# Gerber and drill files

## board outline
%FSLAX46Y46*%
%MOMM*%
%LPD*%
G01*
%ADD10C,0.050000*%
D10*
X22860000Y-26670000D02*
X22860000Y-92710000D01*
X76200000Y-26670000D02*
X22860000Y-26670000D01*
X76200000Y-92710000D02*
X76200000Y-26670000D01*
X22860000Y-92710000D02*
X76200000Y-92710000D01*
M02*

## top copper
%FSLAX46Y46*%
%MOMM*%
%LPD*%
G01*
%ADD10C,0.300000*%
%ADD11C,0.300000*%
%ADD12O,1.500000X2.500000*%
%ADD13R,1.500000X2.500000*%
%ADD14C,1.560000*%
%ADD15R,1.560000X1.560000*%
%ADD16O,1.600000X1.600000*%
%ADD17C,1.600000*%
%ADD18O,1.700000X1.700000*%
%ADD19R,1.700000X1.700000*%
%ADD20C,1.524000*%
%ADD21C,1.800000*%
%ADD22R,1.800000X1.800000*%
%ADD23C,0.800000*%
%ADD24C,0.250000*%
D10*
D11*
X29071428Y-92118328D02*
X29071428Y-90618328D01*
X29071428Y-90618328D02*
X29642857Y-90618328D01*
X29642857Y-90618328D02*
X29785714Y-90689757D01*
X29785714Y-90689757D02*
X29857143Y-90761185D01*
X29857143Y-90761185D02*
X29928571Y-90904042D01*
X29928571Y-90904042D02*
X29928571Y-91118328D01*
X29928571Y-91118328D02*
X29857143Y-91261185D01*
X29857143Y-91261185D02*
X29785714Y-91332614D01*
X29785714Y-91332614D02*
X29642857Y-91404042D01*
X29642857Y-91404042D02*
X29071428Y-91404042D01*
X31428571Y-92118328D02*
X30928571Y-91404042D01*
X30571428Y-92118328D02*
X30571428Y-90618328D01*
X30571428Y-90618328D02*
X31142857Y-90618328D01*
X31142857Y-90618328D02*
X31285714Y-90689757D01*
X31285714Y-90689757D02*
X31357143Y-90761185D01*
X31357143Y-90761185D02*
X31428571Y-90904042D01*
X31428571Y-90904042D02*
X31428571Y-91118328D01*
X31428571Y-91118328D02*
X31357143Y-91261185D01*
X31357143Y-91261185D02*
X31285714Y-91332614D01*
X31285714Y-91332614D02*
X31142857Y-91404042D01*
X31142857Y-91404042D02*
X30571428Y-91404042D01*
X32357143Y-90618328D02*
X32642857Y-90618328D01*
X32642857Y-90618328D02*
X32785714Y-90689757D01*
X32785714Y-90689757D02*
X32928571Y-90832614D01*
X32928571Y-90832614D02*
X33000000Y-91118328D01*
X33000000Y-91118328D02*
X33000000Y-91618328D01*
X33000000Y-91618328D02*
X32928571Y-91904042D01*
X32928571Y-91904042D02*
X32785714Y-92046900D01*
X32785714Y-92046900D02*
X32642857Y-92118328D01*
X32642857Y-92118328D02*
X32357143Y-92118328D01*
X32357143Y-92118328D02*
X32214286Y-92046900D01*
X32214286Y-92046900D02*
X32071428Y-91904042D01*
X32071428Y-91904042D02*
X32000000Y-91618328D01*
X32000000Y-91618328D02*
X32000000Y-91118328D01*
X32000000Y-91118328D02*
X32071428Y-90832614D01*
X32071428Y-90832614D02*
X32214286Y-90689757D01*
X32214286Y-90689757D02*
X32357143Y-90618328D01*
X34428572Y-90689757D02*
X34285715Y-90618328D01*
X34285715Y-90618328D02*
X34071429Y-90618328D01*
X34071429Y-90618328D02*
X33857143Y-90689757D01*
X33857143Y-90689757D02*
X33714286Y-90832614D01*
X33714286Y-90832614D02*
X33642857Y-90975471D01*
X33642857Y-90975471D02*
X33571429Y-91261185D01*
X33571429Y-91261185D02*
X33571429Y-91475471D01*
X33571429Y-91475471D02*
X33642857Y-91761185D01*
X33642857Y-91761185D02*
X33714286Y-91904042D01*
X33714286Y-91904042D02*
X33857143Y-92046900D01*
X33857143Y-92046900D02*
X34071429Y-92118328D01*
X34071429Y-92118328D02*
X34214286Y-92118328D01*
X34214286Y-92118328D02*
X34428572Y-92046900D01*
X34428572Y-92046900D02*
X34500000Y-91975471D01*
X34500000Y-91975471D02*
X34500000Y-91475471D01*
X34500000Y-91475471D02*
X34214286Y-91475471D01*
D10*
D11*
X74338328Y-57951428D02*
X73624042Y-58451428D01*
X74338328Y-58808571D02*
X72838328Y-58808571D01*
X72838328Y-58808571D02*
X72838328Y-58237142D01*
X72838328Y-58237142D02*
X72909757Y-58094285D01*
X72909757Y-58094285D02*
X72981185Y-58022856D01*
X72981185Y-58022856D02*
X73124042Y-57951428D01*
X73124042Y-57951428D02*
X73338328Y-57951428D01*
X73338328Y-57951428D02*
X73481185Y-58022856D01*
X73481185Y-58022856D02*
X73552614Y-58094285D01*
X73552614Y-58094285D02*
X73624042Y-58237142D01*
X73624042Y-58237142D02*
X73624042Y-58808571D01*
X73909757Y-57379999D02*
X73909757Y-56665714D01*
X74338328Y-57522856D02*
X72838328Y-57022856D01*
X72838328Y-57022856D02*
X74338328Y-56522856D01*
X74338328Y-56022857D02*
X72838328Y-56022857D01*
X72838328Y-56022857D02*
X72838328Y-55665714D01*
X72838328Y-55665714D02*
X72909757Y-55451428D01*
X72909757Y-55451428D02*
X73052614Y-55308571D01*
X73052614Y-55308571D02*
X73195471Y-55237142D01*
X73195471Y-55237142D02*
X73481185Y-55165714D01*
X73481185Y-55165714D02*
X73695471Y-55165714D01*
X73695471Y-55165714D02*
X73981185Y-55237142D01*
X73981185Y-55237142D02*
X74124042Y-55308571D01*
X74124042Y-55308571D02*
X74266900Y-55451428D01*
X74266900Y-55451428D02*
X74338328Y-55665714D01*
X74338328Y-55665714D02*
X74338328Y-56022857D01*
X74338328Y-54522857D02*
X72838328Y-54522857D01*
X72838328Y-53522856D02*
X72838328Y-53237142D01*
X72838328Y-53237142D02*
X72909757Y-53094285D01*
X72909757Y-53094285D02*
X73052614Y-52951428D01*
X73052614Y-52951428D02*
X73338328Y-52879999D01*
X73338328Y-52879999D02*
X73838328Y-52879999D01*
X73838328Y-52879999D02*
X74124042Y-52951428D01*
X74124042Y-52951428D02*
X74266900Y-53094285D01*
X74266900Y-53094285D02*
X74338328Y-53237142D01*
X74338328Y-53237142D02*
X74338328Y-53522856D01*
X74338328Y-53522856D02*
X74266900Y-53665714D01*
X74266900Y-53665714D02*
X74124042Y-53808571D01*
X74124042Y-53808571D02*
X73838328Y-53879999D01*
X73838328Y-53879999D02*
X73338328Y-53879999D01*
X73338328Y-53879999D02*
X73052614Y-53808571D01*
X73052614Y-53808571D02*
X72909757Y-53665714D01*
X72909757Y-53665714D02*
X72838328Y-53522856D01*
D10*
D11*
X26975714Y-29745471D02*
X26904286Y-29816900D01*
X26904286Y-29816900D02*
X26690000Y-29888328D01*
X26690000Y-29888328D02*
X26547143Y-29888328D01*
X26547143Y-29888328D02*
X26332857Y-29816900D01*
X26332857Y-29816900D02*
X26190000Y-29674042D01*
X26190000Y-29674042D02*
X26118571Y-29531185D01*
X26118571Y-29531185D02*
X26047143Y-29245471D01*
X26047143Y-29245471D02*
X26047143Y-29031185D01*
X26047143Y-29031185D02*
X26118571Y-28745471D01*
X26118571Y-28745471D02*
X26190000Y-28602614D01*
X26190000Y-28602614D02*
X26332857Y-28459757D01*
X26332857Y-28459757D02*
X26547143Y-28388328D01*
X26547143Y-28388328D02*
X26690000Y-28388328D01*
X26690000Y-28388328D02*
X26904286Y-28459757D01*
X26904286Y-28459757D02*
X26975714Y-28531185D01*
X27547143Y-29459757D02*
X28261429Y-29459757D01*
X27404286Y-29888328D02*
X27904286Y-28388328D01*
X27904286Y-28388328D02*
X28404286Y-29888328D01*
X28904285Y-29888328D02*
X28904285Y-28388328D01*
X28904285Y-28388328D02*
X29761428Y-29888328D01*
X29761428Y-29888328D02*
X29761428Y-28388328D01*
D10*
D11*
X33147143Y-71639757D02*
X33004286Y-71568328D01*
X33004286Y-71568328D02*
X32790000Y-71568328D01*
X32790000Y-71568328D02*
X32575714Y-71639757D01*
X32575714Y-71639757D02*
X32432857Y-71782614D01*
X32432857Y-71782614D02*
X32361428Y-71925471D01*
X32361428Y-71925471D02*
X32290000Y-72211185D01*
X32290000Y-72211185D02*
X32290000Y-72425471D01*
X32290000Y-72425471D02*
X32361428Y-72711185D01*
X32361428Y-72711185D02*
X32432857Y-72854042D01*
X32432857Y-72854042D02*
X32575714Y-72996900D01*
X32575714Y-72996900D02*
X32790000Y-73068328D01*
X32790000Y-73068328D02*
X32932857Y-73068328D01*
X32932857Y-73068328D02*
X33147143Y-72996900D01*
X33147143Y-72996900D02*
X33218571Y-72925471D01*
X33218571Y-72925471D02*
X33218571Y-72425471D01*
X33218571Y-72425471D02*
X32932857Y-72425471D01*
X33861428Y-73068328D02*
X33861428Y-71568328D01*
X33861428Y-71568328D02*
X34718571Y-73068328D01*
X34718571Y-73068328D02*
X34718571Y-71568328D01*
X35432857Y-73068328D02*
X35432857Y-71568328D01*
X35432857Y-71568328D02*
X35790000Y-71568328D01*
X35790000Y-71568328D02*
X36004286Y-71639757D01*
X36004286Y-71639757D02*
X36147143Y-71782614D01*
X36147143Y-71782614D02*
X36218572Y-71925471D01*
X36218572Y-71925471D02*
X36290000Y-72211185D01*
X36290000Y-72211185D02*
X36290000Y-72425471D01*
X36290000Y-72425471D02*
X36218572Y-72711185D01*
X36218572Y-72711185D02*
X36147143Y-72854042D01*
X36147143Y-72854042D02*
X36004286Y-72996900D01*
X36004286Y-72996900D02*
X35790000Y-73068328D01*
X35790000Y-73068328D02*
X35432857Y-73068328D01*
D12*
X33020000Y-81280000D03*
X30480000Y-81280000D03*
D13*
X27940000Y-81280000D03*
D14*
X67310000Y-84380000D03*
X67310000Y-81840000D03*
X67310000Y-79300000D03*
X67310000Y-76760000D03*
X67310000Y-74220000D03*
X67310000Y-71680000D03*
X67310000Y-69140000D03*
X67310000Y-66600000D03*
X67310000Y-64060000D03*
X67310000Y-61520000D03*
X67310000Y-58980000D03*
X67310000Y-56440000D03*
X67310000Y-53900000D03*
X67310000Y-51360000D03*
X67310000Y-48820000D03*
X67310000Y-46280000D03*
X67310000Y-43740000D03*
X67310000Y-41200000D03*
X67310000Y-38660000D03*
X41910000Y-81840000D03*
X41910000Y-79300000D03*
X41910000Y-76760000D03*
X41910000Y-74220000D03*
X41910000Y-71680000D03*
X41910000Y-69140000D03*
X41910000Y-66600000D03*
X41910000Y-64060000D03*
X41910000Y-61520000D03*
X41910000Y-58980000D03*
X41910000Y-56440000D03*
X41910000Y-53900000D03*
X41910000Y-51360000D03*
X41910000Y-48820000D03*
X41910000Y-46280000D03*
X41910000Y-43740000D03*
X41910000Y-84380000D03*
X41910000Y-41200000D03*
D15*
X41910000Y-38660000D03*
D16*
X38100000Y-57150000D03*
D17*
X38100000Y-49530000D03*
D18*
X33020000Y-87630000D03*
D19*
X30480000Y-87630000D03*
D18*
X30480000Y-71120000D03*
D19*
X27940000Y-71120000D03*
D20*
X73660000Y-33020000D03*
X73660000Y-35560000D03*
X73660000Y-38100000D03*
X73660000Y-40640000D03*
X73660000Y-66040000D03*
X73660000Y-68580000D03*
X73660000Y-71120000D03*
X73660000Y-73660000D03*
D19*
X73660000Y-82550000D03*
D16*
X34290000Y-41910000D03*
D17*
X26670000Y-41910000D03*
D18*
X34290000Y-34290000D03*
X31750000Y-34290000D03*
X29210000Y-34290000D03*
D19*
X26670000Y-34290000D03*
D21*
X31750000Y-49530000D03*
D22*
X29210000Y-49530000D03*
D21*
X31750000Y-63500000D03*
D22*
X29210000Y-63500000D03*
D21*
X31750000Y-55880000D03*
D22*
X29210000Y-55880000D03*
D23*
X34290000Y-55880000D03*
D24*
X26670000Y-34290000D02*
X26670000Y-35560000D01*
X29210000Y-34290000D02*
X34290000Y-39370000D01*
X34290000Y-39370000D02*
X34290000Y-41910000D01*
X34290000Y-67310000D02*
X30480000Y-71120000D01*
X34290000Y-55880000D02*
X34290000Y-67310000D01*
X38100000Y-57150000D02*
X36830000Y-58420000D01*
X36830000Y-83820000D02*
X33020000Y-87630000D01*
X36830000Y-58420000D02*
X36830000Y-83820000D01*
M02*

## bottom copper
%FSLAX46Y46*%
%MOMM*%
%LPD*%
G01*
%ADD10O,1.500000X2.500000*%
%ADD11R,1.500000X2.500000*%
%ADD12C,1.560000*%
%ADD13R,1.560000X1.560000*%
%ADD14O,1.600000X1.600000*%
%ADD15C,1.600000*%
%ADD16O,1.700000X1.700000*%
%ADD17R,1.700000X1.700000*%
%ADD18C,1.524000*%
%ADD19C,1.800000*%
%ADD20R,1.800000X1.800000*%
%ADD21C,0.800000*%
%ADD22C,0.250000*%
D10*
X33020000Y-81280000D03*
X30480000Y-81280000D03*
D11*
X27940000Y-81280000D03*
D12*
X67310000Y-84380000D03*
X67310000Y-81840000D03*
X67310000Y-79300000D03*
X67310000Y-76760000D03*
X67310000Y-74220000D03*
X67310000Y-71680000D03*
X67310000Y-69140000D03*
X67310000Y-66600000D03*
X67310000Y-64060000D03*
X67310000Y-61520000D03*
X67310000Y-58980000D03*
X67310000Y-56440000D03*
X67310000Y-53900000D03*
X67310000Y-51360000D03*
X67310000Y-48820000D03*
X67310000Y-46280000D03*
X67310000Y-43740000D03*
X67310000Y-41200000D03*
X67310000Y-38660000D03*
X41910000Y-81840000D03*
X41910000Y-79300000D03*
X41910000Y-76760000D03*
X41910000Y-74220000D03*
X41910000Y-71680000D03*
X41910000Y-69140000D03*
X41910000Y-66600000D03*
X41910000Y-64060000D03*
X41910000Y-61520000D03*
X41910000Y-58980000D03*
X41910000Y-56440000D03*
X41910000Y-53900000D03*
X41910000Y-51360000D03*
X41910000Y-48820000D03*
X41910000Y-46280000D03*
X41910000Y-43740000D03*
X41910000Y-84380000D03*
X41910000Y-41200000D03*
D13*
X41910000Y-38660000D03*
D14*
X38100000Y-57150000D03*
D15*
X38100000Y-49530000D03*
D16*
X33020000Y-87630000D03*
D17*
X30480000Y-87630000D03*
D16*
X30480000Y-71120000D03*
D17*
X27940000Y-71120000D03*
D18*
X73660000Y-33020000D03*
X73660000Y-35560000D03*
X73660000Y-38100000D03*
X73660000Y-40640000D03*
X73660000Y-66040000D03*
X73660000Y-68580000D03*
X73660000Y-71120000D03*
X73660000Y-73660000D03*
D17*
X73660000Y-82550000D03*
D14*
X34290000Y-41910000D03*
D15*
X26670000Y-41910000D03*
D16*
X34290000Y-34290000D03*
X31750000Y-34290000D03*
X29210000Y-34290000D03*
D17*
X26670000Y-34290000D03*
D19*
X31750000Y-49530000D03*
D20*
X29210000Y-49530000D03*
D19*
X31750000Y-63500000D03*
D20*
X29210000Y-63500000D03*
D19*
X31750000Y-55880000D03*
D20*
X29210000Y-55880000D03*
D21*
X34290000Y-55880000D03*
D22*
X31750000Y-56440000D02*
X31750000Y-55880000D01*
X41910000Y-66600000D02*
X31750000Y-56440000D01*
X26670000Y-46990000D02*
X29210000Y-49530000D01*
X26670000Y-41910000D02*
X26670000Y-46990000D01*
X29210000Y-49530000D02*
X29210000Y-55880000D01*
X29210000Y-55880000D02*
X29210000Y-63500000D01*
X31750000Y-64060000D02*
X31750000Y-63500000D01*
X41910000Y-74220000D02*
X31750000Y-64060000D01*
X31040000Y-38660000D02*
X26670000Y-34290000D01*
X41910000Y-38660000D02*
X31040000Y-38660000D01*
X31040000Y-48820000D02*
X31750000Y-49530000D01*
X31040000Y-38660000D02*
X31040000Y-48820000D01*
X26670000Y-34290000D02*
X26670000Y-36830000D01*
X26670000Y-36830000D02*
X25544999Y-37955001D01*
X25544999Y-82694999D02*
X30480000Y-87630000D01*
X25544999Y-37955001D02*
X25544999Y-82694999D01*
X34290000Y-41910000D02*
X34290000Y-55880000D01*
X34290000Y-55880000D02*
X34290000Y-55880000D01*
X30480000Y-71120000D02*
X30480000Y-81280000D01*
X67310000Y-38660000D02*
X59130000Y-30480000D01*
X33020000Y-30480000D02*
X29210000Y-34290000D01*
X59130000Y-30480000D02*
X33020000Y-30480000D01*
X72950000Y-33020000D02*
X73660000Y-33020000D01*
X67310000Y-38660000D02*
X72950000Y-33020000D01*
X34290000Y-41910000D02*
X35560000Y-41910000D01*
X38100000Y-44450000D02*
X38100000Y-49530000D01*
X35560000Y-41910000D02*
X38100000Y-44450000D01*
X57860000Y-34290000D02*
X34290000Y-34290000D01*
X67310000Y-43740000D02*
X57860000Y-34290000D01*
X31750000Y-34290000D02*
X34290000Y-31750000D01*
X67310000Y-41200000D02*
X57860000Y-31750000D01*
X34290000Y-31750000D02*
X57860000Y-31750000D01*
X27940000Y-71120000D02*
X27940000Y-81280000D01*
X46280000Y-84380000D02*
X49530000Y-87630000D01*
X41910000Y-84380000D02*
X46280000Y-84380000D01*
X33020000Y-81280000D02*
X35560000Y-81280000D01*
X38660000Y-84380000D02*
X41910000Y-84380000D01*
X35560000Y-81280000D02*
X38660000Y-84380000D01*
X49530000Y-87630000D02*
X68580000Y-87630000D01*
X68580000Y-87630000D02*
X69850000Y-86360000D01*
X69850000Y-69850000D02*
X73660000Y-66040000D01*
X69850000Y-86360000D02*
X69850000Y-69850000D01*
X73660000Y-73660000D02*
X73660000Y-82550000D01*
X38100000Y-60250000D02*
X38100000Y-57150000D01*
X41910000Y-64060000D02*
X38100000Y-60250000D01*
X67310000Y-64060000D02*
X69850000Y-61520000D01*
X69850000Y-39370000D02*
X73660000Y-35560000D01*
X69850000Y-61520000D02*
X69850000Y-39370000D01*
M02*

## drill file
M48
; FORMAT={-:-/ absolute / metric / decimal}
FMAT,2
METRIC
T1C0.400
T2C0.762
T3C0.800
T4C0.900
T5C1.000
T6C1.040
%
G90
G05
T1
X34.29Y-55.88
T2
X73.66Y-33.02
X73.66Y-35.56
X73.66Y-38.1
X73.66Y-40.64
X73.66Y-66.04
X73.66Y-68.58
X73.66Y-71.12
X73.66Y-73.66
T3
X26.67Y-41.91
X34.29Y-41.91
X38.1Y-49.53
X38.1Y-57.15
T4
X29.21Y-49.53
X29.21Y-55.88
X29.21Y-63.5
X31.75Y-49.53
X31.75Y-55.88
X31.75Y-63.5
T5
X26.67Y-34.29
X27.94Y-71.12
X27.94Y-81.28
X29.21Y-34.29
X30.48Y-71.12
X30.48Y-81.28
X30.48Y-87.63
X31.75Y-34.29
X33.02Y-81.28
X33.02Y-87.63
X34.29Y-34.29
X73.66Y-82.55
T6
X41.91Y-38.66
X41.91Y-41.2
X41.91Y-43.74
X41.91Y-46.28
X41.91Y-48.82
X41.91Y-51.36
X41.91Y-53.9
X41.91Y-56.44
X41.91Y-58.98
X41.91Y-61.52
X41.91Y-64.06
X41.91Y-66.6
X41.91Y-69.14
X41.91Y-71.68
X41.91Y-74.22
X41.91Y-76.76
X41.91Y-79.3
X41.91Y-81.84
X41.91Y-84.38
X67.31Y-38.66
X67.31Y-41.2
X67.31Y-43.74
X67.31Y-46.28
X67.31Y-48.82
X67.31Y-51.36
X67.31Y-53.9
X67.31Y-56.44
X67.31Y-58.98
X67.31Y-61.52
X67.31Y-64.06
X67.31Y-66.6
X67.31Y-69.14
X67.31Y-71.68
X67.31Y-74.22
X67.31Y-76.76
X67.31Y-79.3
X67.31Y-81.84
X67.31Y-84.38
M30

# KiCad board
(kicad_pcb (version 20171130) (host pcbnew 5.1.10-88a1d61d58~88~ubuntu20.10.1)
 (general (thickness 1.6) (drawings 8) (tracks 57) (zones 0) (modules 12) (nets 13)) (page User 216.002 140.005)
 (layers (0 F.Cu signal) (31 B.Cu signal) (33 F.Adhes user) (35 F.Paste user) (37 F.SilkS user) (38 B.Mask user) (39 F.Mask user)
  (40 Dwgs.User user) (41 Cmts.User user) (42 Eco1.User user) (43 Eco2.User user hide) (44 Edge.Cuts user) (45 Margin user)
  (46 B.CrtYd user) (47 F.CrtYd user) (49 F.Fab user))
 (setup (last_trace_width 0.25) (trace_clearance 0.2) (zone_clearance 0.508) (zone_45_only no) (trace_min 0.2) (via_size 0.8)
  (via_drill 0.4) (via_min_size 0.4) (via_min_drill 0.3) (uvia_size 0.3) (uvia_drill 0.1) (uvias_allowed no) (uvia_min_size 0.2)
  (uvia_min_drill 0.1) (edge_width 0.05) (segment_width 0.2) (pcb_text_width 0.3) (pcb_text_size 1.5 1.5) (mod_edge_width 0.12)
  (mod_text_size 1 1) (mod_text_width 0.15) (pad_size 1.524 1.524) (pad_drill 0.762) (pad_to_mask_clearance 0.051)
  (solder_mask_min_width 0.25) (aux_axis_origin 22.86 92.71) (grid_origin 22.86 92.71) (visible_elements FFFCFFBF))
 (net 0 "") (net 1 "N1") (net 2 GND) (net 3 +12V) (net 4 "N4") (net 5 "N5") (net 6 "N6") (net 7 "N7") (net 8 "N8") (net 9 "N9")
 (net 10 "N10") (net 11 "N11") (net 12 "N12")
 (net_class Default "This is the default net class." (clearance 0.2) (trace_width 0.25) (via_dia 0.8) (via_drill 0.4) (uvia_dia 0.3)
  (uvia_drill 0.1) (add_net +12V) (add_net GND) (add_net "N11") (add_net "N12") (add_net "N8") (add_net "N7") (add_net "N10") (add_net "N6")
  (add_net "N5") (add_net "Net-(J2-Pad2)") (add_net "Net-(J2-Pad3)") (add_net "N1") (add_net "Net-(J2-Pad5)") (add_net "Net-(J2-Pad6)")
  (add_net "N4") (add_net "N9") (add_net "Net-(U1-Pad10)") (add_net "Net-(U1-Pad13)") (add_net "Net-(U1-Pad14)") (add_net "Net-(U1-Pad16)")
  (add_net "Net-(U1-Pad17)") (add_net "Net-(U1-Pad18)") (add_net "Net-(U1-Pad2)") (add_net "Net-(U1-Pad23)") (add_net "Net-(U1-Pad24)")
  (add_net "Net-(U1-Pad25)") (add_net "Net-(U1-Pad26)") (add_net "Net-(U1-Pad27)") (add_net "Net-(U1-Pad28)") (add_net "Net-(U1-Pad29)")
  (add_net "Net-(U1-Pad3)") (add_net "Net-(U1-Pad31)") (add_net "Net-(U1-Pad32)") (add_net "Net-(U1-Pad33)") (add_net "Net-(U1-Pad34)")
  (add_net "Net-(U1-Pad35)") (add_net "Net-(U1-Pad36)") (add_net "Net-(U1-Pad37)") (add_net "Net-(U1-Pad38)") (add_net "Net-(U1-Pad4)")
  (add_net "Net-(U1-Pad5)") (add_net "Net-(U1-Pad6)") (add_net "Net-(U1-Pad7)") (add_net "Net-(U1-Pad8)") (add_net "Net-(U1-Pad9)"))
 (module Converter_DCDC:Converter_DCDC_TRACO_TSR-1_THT (layer F.Cu) (at 27.94 81.28)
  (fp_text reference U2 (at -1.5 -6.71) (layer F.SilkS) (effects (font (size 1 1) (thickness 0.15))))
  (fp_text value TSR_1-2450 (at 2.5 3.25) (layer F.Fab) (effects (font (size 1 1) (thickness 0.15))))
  (pad 3 thru_hole oval (at 5.08 0) (size 1.5 2.5) (drill 1) (layers *.Cu *.Mask) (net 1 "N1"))
  (pad 2 thru_hole oval (at 2.54 0) (size 1.5 2.5) (drill 1) (layers *.Cu *.Mask) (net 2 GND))
  (pad 1 thru_hole rect (at 0 0) (size 1.5 2.5) (drill 1) (layers *.Cu *.Mask) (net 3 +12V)))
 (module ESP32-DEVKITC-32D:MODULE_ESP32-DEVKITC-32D (layer F.Cu) (at 54.61 58.42)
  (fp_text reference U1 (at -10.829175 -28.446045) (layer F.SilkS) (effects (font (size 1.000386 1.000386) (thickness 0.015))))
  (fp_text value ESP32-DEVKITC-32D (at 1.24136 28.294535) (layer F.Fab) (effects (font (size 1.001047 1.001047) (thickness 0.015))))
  (pad 38 thru_hole circle (at 12.7 25.96) (size 1.56 1.56) (drill 1.04) (layers *.Cu *.Mask))
  (pad 37 thru_hole circle (at 12.7 23.42) (size 1.56 1.56) (drill 1.04) (layers *.Cu *.Mask))
  (pad 36 thru_hole circle (at 12.7 20.88) (size 1.56 1.56) (drill 1.04) (layers *.Cu *.Mask))
  (pad 35 thru_hole circle (at 12.7 18.34) (size 1.56 1.56) (drill 1.04) (layers *.Cu *.Mask))
  (pad 34 thru_hole circle (at 12.7 15.8) (size 1.56 1.56) (drill 1.04) (layers *.Cu *.Mask))
  (pad 33 thru_hole circle (at 12.7 13.26) (size 1.56 1.56) (drill 1.04) (layers *.Cu *.Mask))
  (pad 32 thru_hole circle (at 12.7 10.72) (size 1.56 1.56) (drill 1.04) (layers *.Cu *.Mask))
  (pad 31 thru_hole circle (at 12.7 8.18) (size 1.56 1.56) (drill 1.04) (layers *.Cu *.Mask))
  (pad 30 thru_hole circle (at 12.7 5.64) (size 1.56 1.56) (drill 1.04) (layers *.Cu *.Mask) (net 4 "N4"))
  (pad 29 thru_hole circle (at 12.7 3.1) (size 1.56 1.56) (drill 1.04) (layers *.Cu *.Mask))
  (pad 28 thru_hole circle (at 12.7 0.56) (size 1.56 1.56) (drill 1.04) (layers *.Cu *.Mask))
  (pad 27 thru_hole circle (at 12.7 -1.98) (size 1.56 1.56) (drill 1.04) (layers *.Cu *.Mask))
  (pad 26 thru_hole circle (at 12.7 -4.52) (size 1.56 1.56) (drill 1.04) (layers *.Cu *.Mask))
  (pad 25 thru_hole circle (at 12.7 -7.06) (size 1.56 1.56) (drill 1.04) (layers *.Cu *.Mask))
  (pad 24 thru_hole circle (at 12.7 -9.6) (size 1.56 1.56) (drill 1.04) (layers *.Cu *.Mask))
  (pad 23 thru_hole circle (at 12.7 -12.14) (size 1.56 1.56) (drill 1.04) (layers *.Cu *.Mask))
  (pad 22 thru_hole circle (at 12.7 -14.68) (size 1.56 1.56) (drill 1.04) (layers *.Cu *.Mask) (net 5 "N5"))
  (pad 21 thru_hole circle (at 12.7 -17.22) (size 1.56 1.56) (drill 1.04) (layers *.Cu *.Mask) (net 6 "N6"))
  (pad 20 thru_hole circle (at 12.7 -19.76) (size 1.56 1.56) (drill 1.04) (layers *.Cu *.Mask) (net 2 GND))
  (pad 18 thru_hole circle (at -12.7 23.42) (size 1.56 1.56) (drill 1.04) (layers *.Cu *.Mask))
  (pad 17 thru_hole circle (at -12.7 20.88) (size 1.56 1.56) (drill 1.04) (layers *.Cu *.Mask))
  (pad 16 thru_hole circle (at -12.7 18.34) (size 1.56 1.56) (drill 1.04) (layers *.Cu *.Mask))
  (pad 15 thru_hole circle (at -12.7 15.8) (size 1.56 1.56) (drill 1.04) (layers *.Cu *.Mask) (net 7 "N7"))
  (pad 14 thru_hole circle (at -12.7 13.26) (size 1.56 1.56) (drill 1.04) (layers *.Cu *.Mask))
  (pad 13 thru_hole circle (at -12.7 10.72) (size 1.56 1.56) (drill 1.04) (layers *.Cu *.Mask))
  (pad 12 thru_hole circle (at -12.7 8.18) (size 1.56 1.56) (drill 1.04) (layers *.Cu *.Mask) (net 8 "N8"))
  (pad 11 thru_hole circle (at -12.7 5.64) (size 1.56 1.56) (drill 1.04) (layers *.Cu *.Mask) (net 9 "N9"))
  (pad 10 thru_hole circle (at -12.7 3.1) (size 1.56 1.56) (drill 1.04) (layers *.Cu *.Mask))
  (pad 9 thru_hole circle (at -12.7 0.56) (size 1.56 1.56) (drill 1.04) (layers *.Cu *.Mask))
  (pad 8 thru_hole circle (at -12.7 -1.98) (size 1.56 1.56) (drill 1.04) (layers *.Cu *.Mask))
  (pad 7 thru_hole circle (at -12.7 -4.52) (size 1.56 1.56) (drill 1.04) (layers *.Cu *.Mask))
  (pad 6 thru_hole circle (at -12.7 -7.06) (size 1.56 1.56) (drill 1.04) (layers *.Cu *.Mask))
  (pad 5 thru_hole circle (at -12.7 -9.6) (size 1.56 1.56) (drill 1.04) (layers *.Cu *.Mask))
  (pad 4 thru_hole circle (at -12.7 -12.14) (size 1.56 1.56) (drill 1.04) (layers *.Cu *.Mask))
  (pad 3 thru_hole circle (at -12.7 -14.68) (size 1.56 1.56) (drill 1.04) (layers *.Cu *.Mask))
  (pad 19 thru_hole circle (at -12.7 25.96) (size 1.56 1.56) (drill 1.04) (layers *.Cu *.Mask) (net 1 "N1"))
  (pad 2 thru_hole circle (at -12.7 -17.22) (size 1.56 1.56) (drill 1.04) (layers *.Cu *.Mask))
  (pad 1 thru_hole rect (at -12.7 -19.76) (size 1.56 1.56) (drill 1.04) (layers *.Cu *.Mask) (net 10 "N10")))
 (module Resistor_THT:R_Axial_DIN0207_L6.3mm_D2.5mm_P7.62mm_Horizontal (layer F.Cu) (at 38.1 49.53 270)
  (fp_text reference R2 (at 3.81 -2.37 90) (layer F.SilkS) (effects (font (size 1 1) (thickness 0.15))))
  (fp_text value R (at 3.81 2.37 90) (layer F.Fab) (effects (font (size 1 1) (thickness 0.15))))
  (pad 2 thru_hole oval (at 7.62 0 270) (size 1.6 1.6) (drill 0.8) (layers *.Cu *.Mask) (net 9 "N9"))
  (pad 1 thru_hole circle (at 0 0 270) (size 1.6 1.6) (drill 0.8) (layers *.Cu *.Mask) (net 2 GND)))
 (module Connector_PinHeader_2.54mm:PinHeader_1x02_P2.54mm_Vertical (layer F.Cu) (at 30.48 87.63 90)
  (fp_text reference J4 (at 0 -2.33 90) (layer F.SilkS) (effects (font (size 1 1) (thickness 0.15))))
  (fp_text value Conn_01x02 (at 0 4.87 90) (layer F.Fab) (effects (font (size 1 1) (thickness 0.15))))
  (pad 2 thru_hole oval (at 0 2.54 90) (size 1.7 1.7) (drill 1) (layers *.Cu *.Mask) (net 9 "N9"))
  (pad 1 thru_hole rect (at 0 0 90) (size 1.7 1.7) (drill 1) (layers *.Cu *.Mask) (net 10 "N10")))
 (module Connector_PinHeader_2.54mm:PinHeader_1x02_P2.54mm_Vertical (layer F.Cu) (at 27.94 71.12 90)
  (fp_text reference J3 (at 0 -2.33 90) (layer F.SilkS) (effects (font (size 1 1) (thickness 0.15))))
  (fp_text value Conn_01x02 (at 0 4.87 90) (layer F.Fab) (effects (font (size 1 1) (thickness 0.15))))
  (pad 2 thru_hole oval (at 0 2.54 90) (size 1.7 1.7) (drill 1) (layers *.Cu *.Mask) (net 2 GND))
  (pad 1 thru_hole rect (at 0 0 90) (size 1.7 1.7) (drill 1) (layers *.Cu *.Mask) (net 3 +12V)))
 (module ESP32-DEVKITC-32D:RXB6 (layer F.Cu) (at 73.66 76.2 180)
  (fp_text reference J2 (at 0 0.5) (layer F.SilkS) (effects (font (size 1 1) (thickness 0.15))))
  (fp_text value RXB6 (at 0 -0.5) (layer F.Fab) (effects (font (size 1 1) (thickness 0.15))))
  (pad 8 thru_hole circle (at 0 43.18 180) (size 1.524 1.524) (drill 0.762) (layers *.Cu *.Mask) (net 2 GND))
  (pad 7 thru_hole circle (at 0 40.64 180) (size 1.524 1.524) (drill 0.762) (layers *.Cu *.Mask) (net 4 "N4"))
  (pad 6 thru_hole circle (at 0 38.1 180) (size 1.524 1.524) (drill 0.762) (layers *.Cu *.Mask))
  (pad 5 thru_hole circle (at 0 35.56 180) (size 1.524 1.524) (drill 0.762) (layers *.Cu *.Mask))
  (pad 4 thru_hole circle (at 0 10.16 180) (size 1.524 1.524) (drill 0.762) (layers *.Cu *.Mask) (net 1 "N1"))
  (pad 3 thru_hole circle (at 0 7.62 180) (size 1.524 1.524) (drill 0.762) (layers *.Cu *.Mask))
  (pad 2 thru_hole circle (at 0 5.08 180) (size 1.524 1.524) (drill 0.762) (layers *.Cu *.Mask))
  (pad 1 thru_hole circle (at 0 2.54 180) (size 1.524 1.524) (drill 0.762) (layers *.Cu *.Mask) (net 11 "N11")))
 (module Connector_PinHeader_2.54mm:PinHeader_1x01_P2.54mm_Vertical (layer F.Cu) (at 73.66 82.55)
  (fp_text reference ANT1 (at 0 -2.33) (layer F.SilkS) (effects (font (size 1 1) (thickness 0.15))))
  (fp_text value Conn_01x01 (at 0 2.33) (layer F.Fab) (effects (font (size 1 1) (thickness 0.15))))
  (pad 1 thru_hole rect (at 0 0) (size 1.7 1.7) (drill 1) (layers *.Cu *.Mask) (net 11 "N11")))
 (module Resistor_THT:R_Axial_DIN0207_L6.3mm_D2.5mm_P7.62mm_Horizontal (layer F.Cu) (at 26.67 41.91)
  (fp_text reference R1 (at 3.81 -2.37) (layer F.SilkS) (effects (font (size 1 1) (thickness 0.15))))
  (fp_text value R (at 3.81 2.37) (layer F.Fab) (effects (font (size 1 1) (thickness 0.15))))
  (pad 2 thru_hole oval (at 7.62 0) (size 1.6 1.6) (drill 0.8) (layers *.Cu *.Mask) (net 2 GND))
  (pad 1 thru_hole circle (at 0 0) (size 1.6 1.6) (drill 0.8) (layers *.Cu *.Mask) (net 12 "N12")))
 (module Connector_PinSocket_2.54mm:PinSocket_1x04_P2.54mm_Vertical (layer F.Cu) (at 26.67 34.29 90)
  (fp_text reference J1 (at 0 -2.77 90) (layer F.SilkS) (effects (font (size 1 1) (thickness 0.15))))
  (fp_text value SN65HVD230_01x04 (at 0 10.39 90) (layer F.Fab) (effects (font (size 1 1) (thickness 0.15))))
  (pad 4 thru_hole oval (at 0 7.62 90) (size 1.7 1.7) (drill 1) (layers *.Cu *.Mask) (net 5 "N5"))
  (pad 3 thru_hole oval (at 0 5.08 90) (size 1.7 1.7) (drill 1) (layers *.Cu *.Mask) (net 6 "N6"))
  (pad 2 thru_hole oval (at 0 2.54 90) (size 1.7 1.7) (drill 1) (layers *.Cu *.Mask) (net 2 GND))
  (pad 1 thru_hole rect (at 0 0 90) (size 1.7 1.7) (drill 1) (layers *.Cu *.Mask) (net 10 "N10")))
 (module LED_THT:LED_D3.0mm (layer F.Cu) (at 29.21 49.53)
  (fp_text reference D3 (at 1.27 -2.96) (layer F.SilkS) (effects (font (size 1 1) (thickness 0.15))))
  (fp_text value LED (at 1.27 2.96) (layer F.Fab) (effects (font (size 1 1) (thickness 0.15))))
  (pad 2 thru_hole circle (at 2.54 0) (size 1.8 1.8) (drill 0.9) (layers *.Cu *.Mask) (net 10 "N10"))
  (pad 1 thru_hole rect (at 0 0) (size 1.8 1.8) (drill 0.9) (layers *.Cu *.Mask) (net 12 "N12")))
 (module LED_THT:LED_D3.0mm (layer F.Cu) (at 29.21 63.5)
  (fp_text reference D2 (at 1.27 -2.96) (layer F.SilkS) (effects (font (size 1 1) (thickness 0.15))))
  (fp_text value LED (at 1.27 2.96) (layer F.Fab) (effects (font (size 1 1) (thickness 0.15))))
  (pad 2 thru_hole circle (at 2.54 0) (size 1.8 1.8) (drill 0.9) (layers *.Cu *.Mask) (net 7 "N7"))
  (pad 1 thru_hole rect (at 0 0) (size 1.8 1.8) (drill 0.9) (layers *.Cu *.Mask) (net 12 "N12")))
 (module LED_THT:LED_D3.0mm (layer F.Cu) (at 29.21 55.88)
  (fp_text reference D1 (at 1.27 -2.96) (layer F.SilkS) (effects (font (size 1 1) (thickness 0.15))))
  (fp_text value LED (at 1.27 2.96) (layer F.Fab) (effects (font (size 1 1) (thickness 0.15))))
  (pad 2 thru_hole circle (at 2.54 0) (size 1.8 1.8) (drill 0.9) (layers *.Cu *.Mask) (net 8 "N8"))
  (pad 1 thru_hole rect (at 0 0) (size 1.8 1.8) (drill 0.9) (layers *.Cu *.Mask) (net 12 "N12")))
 (gr_line (start 22.86 26.67) (end 22.86 92.71) (layer Edge.Cuts) (width 0.05))
 (gr_line (start 76.2 26.67) (end 22.86 26.67) (layer Edge.Cuts) (width 0.05))
 (gr_line (start 76.2 92.71) (end 76.2 26.67) (layer Edge.Cuts) (width 0.05))
 (gr_line (start 22.86 92.71) (end 76.2 92.71) (layer Edge.Cuts) (width 0.05))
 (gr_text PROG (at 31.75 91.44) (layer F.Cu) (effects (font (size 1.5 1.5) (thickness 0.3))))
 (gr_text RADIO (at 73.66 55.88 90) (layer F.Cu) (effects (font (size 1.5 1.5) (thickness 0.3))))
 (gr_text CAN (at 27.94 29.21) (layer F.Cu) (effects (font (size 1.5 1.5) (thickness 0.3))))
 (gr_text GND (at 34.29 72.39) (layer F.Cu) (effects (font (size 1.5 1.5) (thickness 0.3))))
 (segment (start 31.75 56.44) (end 31.75 55.88) (width 0.25) (layer B.Cu) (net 8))
 (segment (start 41.91 66.6) (end 31.75 56.44) (width 0.25) (layer B.Cu) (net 8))
 (segment (start 26.67 46.99) (end 29.21 49.53) (width 0.25) (layer B.Cu) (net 12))
 (segment (start 26.67 41.91) (end 26.67 46.99) (width 0.25) (layer B.Cu) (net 12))
 (segment (start 29.21 49.53) (end 29.21 55.88) (width 0.25) (layer B.Cu) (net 12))
 (segment (start 29.21 55.88) (end 29.21 63.5) (width 0.25) (layer B.Cu) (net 12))
 (segment (start 31.75 64.06) (end 31.75 63.5) (width 0.25) (layer B.Cu) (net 7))
 (segment (start 41.91 74.22) (end 31.75 64.06) (width 0.25) (layer B.Cu) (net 7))
 (segment (start 31.04 38.66) (end 26.67 34.29) (width 0.25) (layer B.Cu) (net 10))
 (segment (start 41.91 38.66) (end 31.04 38.66) (width 0.25) (layer B.Cu) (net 10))
 (segment (start 31.04 48.82) (end 31.75 49.53) (width 0.25) (layer B.Cu) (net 10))
 (segment (start 31.04 38.66) (end 31.04 48.82) (width 0.25) (layer B.Cu) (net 10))
 (segment (start 26.67 34.29) (end 26.67 35.56) (width 0.25) (layer F.Cu) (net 10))
 (segment (start 26.67 34.29) (end 26.67 36.83) (width 0.25) (layer B.Cu) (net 10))
 (segment (start 26.67 36.83) (end 25.544999 37.955001) (width 0.25) (layer B.Cu) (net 10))
 (segment (start 25.544999 82.694999) (end 30.48 87.63) (width 0.25) (layer B.Cu) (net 10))
 (segment (start 25.544999 37.955001) (end 25.544999 82.694999) (width 0.25) (layer B.Cu) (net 10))
 (segment (start 29.21 34.29) (end 34.29 39.37) (width 0.25) (layer F.Cu) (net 2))
 (segment (start 34.29 39.37) (end 34.29 41.91) (width 0.25) (layer F.Cu) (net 2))
 (segment (start 34.29 41.91) (end 34.29 55.88) (width 0.25) (layer B.Cu) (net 2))
 (segment (start 34.29 55.88) (end 34.29 55.88) (width 0.25) (layer B.Cu) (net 2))
 (via (at 34.29 55.88) (size 0.8) (drill 0.4) (layers F.Cu B.Cu) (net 2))
 (segment (start 34.29 67.31) (end 30.48 71.12) (width 0.25) (layer F.Cu) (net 2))
 (segment (start 34.29 55.88) (end 34.29 67.31) (width 0.25) (layer F.Cu) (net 2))
 (segment (start 30.48 71.12) (end 30.48 81.28) (width 0.25) (layer B.Cu) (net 2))
 (segment (start 67.31 38.66) (end 59.13 30.48) (width 0.25) (layer B.Cu) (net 2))
 (segment (start 33.02 30.48) (end 29.21 34.29) (width 0.25) (layer B.Cu) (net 2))
 (segment (start 59.13 30.48) (end 33.02 30.48) (width 0.25) (layer B.Cu) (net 2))
 (segment (start 72.95 33.02) (end 73.66 33.02) (width 0.25) (layer B.Cu) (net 2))
 (segment (start 67.31 38.66) (end 72.95 33.02) (width 0.25) (layer B.Cu) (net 2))
 (segment (start 34.29 41.91) (end 35.56 41.91) (width 0.25) (layer B.Cu) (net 2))
 (segment (start 38.1 44.45) (end 38.1 49.53) (width 0.25) (layer B.Cu) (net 2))
 (segment (start 35.56 41.91) (end 38.1 44.45) (width 0.25) (layer B.Cu) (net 2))
 (segment (start 57.86 34.29) (end 34.29 34.29) (width 0.25) (layer B.Cu) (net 5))
 (segment (start 67.31 43.74) (end 57.86 34.29) (width 0.25) (layer B.Cu) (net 5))
 (segment (start 31.75 34.29) (end 34.29 31.75) (width 0.25) (layer B.Cu) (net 6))
 (segment (start 67.31 41.2) (end 57.86 31.75) (width 0.25) (layer B.Cu) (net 6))
 (segment (start 34.29 31.75) (end 57.86 31.75) (width 0.25) (layer B.Cu) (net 6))
 (segment (start 27.94 71.12) (end 27.94 81.28) (width 0.25) (layer B.Cu) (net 3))
 (segment (start 46.28 84.38) (end 49.53 87.63) (width 0.25) (layer B.Cu) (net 1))
 (segment (start 41.91 84.38) (end 46.28 84.38) (width 0.25) (layer B.Cu) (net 1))
 (segment (start 33.02 81.28) (end 35.56 81.28) (width 0.25) (layer B.Cu) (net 1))
 (segment (start 38.66 84.38) (end 41.91 84.38) (width 0.25) (layer B.Cu) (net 1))
 (segment (start 35.56 81.28) (end 38.66 84.38) (width 0.25) (layer B.Cu) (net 1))
 (segment (start 49.53 87.63) (end 68.58 87.63) (width 0.25) (layer B.Cu) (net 1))
 (segment (start 68.58 87.63) (end 69.85 86.36) (width 0.25) (layer B.Cu) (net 1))
 (segment (start 69.85 69.85) (end 73.66 66.04) (width 0.25) (layer B.Cu) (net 1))
 (segment (start 69.85 86.36) (end 69.85 69.85) (width 0.25) (layer B.Cu) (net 1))
 (segment (start 73.66 73.66) (end 73.66 82.55) (width 0.25) (layer B.Cu) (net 11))
 (segment (start 38.1 60.25) (end 38.1 57.15) (width 0.25) (layer B.Cu) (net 9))
 (segment (start 41.91 64.06) (end 38.1 60.25) (width 0.25) (layer B.Cu) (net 9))
 (segment (start 38.1 57.15) (end 36.83 58.42) (width 0.25) (layer F.Cu) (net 9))
 (segment (start 36.83 83.82) (end 33.02 87.63) (width 0.25) (layer F.Cu) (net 9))
 (segment (start 36.83 58.42) (end 36.83 83.82) (width 0.25) (layer F.Cu) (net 9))
 (segment (start 67.31 64.06) (end 69.85 61.52) (width 0.25) (layer B.Cu) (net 4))
 (segment (start 69.85 39.37) (end 73.66 35.56) (width 0.25) (layer B.Cu) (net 4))
 (segment (start 69.85 61.52) (end 69.85 39.37) (width 0.25) (layer B.Cu) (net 4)))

